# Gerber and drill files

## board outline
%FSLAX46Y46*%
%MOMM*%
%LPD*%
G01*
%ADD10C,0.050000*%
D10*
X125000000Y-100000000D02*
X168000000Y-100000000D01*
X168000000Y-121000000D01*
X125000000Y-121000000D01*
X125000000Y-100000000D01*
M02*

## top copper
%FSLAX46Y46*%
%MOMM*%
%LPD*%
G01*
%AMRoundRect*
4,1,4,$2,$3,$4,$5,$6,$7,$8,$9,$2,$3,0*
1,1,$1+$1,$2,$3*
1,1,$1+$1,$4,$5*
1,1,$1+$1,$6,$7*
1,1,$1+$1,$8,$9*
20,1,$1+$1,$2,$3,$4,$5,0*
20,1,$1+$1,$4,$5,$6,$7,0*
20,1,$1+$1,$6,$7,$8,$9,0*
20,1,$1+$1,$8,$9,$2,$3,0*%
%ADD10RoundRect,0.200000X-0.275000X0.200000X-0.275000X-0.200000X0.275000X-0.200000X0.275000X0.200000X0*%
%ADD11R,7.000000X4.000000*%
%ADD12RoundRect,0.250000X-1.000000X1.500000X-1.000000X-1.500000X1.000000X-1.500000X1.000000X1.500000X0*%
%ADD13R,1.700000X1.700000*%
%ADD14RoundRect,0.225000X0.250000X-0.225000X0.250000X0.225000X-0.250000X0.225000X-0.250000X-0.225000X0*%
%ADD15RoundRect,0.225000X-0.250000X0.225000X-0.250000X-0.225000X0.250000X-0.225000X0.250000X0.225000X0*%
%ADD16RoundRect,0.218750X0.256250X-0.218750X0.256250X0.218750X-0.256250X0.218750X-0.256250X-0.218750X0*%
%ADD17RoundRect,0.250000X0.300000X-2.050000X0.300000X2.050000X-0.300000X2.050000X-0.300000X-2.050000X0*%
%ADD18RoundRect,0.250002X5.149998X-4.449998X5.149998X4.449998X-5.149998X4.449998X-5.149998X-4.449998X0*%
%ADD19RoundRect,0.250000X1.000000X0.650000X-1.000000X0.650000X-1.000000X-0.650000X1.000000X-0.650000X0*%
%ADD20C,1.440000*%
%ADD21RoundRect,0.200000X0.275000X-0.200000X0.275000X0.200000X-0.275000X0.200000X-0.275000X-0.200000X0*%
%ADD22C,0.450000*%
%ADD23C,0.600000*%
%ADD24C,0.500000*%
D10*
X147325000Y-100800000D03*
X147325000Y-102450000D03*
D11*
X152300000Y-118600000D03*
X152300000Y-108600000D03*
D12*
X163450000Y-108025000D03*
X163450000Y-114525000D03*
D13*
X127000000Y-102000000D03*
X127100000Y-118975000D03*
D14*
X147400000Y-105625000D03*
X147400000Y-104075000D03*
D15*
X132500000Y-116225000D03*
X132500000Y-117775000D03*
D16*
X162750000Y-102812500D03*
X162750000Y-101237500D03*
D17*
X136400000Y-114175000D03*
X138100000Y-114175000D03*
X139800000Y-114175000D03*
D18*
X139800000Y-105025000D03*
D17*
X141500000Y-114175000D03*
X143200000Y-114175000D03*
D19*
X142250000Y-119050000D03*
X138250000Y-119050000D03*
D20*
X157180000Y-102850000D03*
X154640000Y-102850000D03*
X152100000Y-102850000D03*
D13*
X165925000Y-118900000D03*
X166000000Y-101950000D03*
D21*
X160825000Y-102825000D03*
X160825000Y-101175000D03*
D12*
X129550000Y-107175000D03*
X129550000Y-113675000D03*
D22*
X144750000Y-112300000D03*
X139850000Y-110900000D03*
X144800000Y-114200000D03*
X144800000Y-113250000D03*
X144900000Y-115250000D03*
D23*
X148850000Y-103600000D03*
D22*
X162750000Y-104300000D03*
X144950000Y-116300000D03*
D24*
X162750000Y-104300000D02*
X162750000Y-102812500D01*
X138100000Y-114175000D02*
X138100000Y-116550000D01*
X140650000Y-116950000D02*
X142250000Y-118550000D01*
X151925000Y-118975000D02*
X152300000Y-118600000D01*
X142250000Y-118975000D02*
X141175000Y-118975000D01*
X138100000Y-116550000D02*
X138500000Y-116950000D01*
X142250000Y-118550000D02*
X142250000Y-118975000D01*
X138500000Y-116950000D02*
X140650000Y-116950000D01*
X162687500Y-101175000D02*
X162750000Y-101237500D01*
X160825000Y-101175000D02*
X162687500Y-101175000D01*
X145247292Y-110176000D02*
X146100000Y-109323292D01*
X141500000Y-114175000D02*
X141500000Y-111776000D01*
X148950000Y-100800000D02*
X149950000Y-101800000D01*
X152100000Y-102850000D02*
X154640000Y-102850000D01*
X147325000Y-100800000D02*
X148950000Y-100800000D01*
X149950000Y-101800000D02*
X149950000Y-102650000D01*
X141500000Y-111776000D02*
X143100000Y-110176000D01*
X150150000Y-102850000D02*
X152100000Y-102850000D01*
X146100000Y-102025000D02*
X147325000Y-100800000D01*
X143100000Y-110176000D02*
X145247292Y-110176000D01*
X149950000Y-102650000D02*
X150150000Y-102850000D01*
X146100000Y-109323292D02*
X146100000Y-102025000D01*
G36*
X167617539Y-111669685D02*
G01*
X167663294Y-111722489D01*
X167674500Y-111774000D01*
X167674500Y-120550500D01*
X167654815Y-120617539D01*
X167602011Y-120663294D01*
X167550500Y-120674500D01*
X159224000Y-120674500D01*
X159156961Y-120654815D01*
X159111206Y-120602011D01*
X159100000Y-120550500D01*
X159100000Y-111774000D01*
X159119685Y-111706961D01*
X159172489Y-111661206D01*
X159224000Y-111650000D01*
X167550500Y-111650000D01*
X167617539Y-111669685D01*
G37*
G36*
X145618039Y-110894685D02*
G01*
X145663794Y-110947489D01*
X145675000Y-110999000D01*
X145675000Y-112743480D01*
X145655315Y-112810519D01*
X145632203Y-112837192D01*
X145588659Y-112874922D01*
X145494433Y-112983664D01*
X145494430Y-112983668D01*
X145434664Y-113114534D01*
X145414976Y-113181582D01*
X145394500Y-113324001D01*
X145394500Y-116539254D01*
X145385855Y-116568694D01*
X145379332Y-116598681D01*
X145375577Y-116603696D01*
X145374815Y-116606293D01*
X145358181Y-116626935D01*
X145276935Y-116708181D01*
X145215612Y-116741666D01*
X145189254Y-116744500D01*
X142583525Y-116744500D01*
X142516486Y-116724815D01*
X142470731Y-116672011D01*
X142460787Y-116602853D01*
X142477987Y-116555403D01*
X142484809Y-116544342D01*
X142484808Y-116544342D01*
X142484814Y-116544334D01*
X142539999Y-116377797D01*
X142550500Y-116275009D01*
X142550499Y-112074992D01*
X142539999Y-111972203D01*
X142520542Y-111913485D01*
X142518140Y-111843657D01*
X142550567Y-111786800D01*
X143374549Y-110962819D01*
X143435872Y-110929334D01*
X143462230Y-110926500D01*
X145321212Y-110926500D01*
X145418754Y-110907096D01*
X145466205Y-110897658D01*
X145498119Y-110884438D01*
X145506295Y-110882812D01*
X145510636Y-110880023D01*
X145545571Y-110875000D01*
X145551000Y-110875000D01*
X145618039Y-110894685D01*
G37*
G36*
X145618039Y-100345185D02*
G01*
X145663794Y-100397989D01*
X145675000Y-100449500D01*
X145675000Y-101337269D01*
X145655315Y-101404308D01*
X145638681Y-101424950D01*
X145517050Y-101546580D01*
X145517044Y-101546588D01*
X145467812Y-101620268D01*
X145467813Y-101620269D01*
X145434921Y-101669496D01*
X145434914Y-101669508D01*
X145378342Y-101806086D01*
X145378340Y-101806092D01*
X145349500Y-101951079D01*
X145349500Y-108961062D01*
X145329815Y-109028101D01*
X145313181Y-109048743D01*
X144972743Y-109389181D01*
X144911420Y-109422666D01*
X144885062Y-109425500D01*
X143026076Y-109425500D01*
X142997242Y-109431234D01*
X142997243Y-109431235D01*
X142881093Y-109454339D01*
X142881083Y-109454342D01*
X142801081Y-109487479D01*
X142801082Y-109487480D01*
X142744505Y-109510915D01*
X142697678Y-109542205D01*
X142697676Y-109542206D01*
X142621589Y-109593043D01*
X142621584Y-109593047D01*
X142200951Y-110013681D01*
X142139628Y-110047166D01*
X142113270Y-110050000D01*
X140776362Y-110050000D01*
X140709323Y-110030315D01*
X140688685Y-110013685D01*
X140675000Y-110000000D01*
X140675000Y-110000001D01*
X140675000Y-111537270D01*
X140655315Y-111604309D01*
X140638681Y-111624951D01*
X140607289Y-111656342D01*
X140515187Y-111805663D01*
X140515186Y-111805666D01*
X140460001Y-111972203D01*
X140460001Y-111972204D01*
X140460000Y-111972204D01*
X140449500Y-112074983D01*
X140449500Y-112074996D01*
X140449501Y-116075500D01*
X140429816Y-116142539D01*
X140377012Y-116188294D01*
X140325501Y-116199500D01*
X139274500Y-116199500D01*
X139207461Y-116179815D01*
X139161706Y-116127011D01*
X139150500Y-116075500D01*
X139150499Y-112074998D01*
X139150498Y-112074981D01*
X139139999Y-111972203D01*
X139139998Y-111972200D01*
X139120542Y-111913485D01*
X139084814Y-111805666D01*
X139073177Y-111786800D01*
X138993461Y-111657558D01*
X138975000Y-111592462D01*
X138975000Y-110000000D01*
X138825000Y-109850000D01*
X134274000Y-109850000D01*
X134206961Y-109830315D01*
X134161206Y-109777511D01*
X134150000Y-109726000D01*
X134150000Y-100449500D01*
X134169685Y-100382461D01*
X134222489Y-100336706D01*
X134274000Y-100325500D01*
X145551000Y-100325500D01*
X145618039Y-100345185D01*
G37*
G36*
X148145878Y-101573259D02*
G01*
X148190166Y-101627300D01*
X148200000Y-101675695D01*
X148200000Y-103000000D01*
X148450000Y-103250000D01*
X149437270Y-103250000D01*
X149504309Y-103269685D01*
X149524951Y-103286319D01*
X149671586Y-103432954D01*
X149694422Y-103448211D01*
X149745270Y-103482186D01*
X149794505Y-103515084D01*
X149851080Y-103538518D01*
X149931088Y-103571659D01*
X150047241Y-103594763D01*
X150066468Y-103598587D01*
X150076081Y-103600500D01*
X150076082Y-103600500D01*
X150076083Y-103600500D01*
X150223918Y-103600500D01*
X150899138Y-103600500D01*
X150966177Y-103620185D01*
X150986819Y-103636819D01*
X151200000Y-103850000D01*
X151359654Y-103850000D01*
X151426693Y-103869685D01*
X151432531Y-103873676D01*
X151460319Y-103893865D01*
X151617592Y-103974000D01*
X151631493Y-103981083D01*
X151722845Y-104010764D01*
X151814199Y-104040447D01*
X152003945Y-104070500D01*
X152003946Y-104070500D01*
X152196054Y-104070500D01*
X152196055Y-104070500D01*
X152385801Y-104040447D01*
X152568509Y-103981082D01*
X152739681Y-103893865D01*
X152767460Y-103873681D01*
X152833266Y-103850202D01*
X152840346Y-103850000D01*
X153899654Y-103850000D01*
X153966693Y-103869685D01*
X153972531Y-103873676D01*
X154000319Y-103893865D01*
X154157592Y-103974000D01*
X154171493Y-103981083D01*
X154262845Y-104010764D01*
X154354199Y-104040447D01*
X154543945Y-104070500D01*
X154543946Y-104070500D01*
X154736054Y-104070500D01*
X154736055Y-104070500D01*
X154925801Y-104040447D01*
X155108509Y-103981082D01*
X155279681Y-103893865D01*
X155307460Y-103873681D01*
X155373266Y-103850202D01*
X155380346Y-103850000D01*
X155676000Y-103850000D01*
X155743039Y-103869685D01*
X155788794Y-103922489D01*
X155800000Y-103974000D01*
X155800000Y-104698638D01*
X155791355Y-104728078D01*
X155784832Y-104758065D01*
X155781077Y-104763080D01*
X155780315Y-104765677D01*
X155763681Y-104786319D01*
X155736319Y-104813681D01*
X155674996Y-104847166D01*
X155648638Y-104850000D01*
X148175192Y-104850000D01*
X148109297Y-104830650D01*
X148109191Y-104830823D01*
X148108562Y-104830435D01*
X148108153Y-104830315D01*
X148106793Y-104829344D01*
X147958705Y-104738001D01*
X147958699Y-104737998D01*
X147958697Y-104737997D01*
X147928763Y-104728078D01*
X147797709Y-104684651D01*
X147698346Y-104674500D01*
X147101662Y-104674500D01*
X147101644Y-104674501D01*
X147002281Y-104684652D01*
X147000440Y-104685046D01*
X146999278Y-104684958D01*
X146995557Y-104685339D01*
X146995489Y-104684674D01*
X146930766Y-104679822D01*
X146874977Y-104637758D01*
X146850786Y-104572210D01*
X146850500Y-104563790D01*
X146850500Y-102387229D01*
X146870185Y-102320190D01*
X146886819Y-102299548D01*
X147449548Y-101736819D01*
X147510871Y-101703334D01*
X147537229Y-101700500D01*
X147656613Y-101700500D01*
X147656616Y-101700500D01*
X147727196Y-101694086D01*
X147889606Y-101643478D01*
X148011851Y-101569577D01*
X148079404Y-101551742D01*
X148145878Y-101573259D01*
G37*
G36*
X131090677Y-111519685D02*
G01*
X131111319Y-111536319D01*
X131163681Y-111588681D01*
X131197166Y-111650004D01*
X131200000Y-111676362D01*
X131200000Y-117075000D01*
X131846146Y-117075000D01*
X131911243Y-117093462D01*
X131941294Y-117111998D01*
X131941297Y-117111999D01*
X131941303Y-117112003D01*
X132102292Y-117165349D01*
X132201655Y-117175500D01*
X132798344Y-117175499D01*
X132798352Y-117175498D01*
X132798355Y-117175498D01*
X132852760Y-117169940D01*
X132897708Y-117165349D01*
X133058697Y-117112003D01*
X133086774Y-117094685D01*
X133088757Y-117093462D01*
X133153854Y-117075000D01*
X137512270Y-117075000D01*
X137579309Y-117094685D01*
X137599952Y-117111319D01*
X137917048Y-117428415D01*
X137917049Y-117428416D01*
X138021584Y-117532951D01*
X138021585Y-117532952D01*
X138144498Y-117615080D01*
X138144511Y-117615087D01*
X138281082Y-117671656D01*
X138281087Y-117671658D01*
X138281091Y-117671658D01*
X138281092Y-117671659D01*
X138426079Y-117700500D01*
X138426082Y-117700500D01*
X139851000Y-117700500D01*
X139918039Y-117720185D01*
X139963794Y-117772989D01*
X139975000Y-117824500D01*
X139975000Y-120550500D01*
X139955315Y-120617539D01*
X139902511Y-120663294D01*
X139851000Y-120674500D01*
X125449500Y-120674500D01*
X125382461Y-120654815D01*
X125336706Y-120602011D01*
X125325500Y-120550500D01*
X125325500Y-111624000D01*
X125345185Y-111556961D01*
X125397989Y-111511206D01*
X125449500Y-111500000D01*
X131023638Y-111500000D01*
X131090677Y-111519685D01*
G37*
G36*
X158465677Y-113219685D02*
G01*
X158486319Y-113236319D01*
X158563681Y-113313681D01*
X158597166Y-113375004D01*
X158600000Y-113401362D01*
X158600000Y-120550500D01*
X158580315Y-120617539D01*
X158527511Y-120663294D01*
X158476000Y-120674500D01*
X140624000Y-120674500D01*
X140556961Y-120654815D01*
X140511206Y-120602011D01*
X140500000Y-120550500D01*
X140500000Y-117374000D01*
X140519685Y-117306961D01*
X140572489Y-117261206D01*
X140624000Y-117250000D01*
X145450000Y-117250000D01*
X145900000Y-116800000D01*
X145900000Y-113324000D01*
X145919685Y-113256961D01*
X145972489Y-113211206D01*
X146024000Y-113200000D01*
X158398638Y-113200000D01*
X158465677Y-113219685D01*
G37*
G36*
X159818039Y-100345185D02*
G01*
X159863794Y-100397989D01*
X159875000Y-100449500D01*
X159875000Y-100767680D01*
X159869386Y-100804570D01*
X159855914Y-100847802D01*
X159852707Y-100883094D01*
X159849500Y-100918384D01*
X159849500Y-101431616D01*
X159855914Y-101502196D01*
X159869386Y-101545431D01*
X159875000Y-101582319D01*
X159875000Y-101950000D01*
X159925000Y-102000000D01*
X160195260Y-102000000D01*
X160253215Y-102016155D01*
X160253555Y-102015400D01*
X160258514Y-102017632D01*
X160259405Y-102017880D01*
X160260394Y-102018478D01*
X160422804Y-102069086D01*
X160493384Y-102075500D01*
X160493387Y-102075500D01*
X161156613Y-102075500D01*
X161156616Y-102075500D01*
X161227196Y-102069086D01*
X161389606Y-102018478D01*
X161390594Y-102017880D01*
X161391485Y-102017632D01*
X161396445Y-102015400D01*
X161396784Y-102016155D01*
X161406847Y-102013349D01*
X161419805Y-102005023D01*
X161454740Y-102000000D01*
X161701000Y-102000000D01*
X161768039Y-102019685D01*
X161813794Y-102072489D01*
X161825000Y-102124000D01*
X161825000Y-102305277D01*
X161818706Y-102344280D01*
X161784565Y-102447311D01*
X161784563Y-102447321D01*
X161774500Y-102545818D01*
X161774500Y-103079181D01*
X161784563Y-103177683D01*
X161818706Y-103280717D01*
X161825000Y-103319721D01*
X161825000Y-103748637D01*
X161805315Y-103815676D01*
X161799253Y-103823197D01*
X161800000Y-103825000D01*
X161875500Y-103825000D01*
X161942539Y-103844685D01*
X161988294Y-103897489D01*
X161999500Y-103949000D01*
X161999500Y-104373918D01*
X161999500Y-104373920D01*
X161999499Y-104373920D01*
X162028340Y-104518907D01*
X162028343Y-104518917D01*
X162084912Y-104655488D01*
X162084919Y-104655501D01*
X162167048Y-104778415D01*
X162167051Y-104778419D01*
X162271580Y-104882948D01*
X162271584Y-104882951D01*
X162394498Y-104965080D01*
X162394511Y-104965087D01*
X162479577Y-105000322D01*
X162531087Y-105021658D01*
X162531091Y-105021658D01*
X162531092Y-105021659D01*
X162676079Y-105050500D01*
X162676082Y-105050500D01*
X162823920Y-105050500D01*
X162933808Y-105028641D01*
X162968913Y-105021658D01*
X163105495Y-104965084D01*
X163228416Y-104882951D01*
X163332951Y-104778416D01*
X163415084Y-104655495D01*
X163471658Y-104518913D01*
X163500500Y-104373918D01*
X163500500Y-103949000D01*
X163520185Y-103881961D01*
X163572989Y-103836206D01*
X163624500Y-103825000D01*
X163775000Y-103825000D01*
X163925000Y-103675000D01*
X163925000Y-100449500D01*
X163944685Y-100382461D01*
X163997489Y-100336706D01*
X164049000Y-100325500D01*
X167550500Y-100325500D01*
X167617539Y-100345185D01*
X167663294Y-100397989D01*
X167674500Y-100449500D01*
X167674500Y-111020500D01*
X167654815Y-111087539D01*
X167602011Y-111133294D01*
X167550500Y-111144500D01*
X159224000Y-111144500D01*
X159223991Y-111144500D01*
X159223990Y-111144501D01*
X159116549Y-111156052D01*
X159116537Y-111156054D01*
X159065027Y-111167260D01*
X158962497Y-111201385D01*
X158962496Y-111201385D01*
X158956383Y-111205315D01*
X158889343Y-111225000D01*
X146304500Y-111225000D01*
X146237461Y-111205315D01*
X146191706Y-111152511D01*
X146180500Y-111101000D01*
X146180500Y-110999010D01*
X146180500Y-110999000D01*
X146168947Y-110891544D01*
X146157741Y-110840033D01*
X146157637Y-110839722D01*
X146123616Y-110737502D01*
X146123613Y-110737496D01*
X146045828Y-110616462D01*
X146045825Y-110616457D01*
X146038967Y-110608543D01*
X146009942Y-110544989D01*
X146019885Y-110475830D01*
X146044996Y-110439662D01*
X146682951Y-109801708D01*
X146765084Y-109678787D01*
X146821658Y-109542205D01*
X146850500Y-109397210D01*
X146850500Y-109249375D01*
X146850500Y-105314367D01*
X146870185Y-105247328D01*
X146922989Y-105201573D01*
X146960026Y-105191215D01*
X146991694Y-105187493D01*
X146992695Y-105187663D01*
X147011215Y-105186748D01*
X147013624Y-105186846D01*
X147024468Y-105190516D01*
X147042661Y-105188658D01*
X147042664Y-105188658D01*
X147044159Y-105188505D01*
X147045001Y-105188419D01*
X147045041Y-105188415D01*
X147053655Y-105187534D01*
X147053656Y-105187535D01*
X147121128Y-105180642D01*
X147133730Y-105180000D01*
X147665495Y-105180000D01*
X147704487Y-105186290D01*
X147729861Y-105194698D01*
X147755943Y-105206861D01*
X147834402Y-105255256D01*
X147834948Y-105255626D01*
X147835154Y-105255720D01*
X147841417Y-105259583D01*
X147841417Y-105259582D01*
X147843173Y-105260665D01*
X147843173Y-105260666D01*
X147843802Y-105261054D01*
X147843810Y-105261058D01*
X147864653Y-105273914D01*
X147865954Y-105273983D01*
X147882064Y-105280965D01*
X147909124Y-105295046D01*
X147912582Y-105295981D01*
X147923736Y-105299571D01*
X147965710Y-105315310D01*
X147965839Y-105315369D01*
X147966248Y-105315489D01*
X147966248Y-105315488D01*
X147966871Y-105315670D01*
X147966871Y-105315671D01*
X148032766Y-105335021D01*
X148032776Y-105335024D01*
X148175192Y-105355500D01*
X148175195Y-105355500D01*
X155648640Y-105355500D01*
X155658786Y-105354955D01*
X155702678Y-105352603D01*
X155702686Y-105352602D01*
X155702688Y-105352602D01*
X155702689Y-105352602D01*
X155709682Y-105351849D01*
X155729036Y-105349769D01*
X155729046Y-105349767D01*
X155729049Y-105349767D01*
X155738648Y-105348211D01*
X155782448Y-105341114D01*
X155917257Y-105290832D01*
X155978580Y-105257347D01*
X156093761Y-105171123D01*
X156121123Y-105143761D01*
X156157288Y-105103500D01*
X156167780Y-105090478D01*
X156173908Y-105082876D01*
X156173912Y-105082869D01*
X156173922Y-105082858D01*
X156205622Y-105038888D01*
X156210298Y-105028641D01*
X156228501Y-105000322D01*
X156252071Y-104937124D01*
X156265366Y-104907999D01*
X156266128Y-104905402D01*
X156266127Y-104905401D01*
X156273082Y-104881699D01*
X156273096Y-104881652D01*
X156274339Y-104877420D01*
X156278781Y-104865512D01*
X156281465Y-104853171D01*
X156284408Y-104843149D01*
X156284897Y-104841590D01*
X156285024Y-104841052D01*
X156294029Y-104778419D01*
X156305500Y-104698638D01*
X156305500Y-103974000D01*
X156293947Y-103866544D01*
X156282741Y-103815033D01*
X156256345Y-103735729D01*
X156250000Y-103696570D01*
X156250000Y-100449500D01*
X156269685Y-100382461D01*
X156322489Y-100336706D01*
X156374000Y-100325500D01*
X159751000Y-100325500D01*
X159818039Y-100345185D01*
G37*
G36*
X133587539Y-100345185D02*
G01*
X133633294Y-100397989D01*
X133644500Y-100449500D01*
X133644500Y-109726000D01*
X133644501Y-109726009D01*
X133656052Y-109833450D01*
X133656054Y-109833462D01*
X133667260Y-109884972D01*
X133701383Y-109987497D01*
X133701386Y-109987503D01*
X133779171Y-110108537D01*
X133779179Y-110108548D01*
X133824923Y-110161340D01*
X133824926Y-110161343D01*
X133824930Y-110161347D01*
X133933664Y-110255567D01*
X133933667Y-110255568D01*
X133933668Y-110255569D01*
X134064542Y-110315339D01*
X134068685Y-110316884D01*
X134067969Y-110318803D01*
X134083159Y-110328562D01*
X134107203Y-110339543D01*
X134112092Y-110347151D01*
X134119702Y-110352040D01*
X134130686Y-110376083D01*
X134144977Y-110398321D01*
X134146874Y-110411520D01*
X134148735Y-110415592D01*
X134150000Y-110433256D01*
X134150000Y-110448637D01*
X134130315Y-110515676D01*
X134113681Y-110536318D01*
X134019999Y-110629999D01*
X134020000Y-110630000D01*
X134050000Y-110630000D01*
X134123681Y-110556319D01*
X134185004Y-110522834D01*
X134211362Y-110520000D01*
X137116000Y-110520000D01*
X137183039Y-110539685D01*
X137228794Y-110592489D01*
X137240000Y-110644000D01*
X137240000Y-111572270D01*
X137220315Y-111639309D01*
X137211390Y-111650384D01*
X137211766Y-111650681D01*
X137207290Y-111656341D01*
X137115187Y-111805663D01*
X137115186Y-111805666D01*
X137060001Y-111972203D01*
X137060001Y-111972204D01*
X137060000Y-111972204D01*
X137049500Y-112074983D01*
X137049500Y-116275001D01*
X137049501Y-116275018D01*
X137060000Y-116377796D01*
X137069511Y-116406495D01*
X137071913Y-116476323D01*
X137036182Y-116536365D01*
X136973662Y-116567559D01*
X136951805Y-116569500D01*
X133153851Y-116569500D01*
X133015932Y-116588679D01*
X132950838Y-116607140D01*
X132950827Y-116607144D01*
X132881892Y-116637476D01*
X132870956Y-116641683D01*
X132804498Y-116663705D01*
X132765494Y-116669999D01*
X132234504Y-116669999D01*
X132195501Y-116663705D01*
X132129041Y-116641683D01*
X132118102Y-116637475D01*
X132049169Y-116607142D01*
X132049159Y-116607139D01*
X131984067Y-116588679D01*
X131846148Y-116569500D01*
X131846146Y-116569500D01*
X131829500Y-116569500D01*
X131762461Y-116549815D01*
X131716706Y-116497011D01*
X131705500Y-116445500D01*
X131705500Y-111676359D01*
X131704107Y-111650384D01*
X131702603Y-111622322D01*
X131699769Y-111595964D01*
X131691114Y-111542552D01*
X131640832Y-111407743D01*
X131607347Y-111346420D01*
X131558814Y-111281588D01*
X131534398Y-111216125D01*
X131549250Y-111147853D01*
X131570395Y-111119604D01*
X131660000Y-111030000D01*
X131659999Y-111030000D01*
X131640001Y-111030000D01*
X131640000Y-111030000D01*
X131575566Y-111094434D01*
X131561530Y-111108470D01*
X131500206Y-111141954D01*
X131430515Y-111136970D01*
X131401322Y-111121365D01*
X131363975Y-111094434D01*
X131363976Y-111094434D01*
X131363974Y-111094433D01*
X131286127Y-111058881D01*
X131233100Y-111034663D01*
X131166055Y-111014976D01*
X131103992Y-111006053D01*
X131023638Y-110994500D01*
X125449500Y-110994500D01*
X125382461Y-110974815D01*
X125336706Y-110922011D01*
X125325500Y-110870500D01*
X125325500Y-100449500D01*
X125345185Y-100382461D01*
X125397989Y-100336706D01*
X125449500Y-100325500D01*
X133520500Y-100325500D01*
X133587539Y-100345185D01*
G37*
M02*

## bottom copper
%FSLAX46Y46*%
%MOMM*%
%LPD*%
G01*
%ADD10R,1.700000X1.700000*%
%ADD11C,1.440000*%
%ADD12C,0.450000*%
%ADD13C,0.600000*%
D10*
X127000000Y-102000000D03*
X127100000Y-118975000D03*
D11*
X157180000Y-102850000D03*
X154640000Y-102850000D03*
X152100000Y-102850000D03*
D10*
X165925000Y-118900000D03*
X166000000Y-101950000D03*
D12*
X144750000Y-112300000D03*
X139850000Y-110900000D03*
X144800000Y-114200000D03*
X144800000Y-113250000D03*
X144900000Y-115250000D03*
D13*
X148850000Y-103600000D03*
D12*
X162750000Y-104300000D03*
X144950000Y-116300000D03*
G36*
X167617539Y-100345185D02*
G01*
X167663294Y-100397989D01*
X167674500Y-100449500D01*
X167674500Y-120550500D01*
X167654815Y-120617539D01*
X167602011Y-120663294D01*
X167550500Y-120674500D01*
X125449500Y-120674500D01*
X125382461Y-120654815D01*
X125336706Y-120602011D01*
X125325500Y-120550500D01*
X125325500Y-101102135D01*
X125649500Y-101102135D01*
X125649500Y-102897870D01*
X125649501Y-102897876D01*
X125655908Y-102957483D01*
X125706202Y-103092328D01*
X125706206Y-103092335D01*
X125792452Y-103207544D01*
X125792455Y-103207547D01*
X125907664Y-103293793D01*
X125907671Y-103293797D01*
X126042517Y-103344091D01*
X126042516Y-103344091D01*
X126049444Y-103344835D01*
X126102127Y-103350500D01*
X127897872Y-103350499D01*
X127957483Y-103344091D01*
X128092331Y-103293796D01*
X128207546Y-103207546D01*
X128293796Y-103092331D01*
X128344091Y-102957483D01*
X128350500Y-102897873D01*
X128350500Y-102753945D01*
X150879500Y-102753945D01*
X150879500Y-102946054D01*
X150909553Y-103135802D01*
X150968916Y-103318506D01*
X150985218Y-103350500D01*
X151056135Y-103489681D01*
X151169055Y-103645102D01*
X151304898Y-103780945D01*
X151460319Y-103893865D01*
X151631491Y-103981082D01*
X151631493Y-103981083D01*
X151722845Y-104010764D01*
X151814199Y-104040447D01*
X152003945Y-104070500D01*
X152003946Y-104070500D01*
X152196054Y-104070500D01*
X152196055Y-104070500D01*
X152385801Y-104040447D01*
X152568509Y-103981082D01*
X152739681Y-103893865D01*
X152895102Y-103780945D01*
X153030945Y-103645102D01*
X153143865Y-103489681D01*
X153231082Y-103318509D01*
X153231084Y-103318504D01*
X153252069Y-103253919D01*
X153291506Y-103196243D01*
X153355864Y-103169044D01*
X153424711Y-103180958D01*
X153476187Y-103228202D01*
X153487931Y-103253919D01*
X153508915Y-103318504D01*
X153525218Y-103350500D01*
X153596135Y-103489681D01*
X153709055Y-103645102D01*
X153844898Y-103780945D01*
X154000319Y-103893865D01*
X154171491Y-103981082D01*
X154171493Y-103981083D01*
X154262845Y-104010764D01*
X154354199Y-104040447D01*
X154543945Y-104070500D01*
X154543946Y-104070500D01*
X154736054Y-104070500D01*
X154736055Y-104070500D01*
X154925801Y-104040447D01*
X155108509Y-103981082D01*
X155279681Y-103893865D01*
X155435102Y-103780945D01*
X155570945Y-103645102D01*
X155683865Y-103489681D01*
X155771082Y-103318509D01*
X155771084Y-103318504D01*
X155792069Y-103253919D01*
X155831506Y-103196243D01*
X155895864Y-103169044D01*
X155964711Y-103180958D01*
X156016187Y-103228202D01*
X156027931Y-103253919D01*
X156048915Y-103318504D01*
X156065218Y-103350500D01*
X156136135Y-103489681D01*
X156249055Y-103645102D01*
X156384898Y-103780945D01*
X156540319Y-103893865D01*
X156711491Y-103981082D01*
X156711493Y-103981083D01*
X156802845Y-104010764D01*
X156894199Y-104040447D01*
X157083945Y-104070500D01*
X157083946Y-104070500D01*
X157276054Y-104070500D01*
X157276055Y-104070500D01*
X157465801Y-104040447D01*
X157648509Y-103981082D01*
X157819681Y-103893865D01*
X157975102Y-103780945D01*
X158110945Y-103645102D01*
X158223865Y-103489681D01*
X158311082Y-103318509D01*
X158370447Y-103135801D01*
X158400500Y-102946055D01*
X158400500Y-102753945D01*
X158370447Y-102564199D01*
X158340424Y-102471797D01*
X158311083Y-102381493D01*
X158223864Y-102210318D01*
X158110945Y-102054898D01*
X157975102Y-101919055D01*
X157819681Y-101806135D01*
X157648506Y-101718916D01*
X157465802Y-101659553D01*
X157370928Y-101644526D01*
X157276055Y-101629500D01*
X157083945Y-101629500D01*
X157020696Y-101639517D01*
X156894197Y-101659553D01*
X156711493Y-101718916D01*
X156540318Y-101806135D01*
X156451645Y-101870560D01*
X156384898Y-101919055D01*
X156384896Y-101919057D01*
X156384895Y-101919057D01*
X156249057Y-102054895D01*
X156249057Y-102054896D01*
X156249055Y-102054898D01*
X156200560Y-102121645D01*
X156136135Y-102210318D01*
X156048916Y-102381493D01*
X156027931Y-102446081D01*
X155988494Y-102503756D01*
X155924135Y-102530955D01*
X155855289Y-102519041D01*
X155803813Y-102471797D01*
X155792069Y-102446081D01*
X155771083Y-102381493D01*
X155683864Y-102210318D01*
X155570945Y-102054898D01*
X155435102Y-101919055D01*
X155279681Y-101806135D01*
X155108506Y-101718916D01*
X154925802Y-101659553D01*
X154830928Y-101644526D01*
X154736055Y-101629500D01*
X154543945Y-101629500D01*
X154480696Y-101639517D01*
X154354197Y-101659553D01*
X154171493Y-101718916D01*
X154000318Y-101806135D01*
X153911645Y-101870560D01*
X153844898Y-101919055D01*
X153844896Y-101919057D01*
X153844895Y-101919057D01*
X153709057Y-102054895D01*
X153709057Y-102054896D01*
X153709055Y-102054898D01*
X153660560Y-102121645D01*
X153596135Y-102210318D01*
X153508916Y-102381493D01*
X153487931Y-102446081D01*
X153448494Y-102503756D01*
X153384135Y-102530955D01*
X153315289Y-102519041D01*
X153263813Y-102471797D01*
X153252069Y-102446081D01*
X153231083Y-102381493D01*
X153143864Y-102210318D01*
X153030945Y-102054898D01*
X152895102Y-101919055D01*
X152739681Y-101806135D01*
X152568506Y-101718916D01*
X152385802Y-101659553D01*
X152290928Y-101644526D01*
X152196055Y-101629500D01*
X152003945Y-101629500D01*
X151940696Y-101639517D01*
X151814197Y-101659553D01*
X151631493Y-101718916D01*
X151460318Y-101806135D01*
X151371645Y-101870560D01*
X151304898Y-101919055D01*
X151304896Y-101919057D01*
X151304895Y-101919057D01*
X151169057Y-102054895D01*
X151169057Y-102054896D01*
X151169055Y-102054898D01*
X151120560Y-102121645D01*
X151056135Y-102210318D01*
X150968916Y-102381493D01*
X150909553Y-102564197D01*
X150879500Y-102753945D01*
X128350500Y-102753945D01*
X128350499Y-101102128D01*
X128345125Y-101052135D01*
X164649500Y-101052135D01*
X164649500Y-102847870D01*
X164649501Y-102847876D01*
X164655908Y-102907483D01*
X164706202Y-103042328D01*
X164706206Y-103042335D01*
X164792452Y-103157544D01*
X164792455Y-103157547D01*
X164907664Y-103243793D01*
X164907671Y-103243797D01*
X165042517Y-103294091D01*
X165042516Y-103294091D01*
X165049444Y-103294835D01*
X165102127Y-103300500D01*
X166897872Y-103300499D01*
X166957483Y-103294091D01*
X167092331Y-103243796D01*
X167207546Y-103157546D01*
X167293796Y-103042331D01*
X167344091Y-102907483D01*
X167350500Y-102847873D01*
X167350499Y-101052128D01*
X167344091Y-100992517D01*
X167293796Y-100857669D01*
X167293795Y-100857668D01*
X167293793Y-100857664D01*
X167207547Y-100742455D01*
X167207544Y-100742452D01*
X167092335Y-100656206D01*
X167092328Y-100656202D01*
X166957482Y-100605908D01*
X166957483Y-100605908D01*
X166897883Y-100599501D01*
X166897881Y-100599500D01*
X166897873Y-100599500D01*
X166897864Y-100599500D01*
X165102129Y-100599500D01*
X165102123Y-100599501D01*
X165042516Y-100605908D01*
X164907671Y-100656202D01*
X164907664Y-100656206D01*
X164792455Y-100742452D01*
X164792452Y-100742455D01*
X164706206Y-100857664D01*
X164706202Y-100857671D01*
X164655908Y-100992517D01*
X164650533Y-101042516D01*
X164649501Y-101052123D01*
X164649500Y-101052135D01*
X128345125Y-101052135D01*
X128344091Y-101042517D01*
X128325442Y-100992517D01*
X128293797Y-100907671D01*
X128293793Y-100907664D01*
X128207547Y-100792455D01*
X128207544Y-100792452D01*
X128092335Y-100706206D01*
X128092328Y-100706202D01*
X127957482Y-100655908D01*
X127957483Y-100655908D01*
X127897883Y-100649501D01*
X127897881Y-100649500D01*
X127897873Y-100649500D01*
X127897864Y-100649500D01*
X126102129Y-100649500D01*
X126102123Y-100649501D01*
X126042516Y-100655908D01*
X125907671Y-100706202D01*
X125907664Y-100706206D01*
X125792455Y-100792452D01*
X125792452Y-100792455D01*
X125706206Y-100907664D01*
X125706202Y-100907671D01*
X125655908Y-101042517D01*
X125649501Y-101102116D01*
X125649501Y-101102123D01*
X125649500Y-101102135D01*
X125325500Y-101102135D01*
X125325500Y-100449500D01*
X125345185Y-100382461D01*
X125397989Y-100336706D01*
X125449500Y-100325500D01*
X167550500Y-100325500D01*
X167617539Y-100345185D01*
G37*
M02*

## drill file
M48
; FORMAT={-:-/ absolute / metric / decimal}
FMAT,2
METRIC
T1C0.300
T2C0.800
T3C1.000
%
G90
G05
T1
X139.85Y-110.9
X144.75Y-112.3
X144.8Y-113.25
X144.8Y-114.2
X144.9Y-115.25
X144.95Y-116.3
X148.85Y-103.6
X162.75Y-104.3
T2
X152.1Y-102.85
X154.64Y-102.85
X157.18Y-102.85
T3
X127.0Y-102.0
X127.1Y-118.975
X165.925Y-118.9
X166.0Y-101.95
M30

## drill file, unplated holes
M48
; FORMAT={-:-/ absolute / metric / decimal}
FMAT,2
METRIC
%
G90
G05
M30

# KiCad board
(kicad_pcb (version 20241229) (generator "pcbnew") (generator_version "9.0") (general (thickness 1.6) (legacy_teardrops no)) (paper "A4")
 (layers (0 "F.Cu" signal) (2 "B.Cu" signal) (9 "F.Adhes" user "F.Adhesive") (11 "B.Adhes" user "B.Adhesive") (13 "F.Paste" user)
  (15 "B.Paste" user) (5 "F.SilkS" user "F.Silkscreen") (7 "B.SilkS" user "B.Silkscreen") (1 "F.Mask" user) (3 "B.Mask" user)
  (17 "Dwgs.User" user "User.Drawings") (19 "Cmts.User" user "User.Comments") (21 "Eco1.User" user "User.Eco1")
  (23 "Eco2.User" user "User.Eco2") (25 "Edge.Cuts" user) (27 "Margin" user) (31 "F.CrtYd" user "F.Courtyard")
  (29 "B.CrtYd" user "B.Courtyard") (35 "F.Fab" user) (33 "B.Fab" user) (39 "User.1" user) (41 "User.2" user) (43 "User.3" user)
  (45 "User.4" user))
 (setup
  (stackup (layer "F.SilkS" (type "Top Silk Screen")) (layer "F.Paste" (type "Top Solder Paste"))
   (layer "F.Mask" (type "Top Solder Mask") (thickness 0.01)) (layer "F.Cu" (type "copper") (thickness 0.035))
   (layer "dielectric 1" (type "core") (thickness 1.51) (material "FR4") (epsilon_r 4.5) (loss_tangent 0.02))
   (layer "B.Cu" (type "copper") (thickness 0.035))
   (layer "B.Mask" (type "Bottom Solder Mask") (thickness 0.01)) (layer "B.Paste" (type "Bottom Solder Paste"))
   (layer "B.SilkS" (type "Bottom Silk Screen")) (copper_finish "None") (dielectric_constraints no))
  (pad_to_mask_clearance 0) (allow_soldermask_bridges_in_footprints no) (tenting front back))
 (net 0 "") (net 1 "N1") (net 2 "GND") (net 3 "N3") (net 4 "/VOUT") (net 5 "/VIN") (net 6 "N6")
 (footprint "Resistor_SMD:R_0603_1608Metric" (layer "F.Cu") (at 147.325 101.625 -90)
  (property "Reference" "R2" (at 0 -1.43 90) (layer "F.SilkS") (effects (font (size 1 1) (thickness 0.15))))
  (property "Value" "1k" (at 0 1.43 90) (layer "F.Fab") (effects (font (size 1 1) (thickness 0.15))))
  (pad "1" smd roundrect (at -0.825 0 270) (size 0.8 0.95) (layers "F.Cu" "F.Mask" "F.Paste") (roundrect_rratio 0.25) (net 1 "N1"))
  (pad "2" smd roundrect (at 0.825 0 270) (size 0.8 0.95) (layers "F.Cu" "F.Mask" "F.Paste") (roundrect_rratio 0.25) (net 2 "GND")))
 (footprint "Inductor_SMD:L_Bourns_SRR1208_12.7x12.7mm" (layer "F.Cu") (at 152.3 113.6 90)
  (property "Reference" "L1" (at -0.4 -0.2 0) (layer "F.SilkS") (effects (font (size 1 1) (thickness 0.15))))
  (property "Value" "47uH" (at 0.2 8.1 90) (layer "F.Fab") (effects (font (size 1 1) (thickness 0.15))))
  (pad "1" smd rect (at -5 0 90) (size 4 7) (layers "F.Cu" "F.Mask" "F.Paste") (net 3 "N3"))
  (pad "2" smd rect (at 5 0 90) (size 4 7) (layers "F.Cu" "F.Mask" "F.Paste") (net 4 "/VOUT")))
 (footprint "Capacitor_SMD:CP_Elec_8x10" (layer "F.Cu") (at 163.45 111.275 -90)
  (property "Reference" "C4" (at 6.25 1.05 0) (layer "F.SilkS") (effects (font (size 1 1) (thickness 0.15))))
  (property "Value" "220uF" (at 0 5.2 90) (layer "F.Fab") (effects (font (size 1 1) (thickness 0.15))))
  (pad "1" smd roundrect (at -3.25 0 270) (size 3.5 2.5) (layers "F.Cu" "F.Mask" "F.Paste") (roundrect_rratio 0.1) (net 4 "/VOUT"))
  (pad "2" smd roundrect (at 3.25 0 270) (size 3.5 2.5) (layers "F.Cu" "F.Mask" "F.Paste") (roundrect_rratio 0.1) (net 2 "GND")))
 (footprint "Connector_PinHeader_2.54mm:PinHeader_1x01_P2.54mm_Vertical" (layer "F.Cu") (at 127 102)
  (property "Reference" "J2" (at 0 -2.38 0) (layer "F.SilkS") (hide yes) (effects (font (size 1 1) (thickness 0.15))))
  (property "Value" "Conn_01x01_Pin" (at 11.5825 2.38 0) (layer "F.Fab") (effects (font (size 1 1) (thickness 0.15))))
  (pad "1" thru_hole rect (at 0 0) (size 1.7 1.7) (drill 1) (layers "*.Cu" "*.Mask") (remove_unused_layers no) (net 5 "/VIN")))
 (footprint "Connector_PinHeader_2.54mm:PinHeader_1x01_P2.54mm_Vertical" (layer "F.Cu") (at 127.1 118.975)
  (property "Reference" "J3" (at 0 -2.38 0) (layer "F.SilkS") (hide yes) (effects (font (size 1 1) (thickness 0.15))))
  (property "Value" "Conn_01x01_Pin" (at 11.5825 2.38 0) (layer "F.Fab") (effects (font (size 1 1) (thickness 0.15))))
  (pad "1" thru_hole rect (at 0 0) (size 1.7 1.7) (drill 1) (layers "*.Cu" "*.Mask") (remove_unused_layers no) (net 2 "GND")))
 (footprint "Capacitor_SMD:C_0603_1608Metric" (layer "F.Cu") (at 147.4 104.85 90)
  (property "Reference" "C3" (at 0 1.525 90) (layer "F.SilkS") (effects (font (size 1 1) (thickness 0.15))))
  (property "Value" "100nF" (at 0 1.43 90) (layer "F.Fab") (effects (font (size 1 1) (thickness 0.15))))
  (pad "1" smd roundrect (at -0.775 0 90) (size 0.9 0.95) (layers "F.Cu" "F.Mask" "F.Paste") (roundrect_rratio 0.25) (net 4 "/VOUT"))
  (pad "2" smd roundrect (at 0.775 0 90) (size 0.9 0.95) (layers "F.Cu" "F.Mask" "F.Paste") (roundrect_rratio 0.25) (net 2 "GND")))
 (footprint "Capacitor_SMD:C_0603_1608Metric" (layer "F.Cu") (at 132.5 117 -90)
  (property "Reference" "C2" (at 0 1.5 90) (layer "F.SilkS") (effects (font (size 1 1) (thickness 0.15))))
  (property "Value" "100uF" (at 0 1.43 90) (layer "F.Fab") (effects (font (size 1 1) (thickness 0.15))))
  (pad "1" smd roundrect (at -0.775 0 270) (size 0.9 0.95) (layers "F.Cu" "F.Mask" "F.Paste") (roundrect_rratio 0.25) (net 5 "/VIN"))
  (pad "2" smd roundrect (at 0.775 0 270) (size 0.9 0.95) (layers "F.Cu" "F.Mask" "F.Paste") (roundrect_rratio 0.25) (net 2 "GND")))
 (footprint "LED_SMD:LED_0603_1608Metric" (layer "F.Cu") (at 162.75 102.025 90)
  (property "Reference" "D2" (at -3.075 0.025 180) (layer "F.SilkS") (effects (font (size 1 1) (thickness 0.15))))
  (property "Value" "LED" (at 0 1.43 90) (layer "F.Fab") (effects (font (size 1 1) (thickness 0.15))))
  (pad "1" smd roundrect (at -0.7875 0 90) (size 0.875 0.95) (layers "F.Cu" "F.Mask" "F.Paste") (roundrect_rratio 0.25) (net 2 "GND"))
  (pad "2" smd roundrect (at 0.7875 0 90) (size 0.875 0.95) (layers "F.Cu" "F.Mask" "F.Paste") (roundrect_rratio 0.25) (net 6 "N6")))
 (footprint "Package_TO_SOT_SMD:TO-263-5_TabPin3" (layer "F.Cu") (at 139.8 106.525 90)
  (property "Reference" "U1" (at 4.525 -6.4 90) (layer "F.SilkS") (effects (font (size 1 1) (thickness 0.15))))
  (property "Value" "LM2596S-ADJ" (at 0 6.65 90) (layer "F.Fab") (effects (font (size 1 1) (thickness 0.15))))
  (pad "" smd roundrect (at -0.925 -2.775 90) (size 4.55 5.25) (layers "F.Paste") (roundrect_rratio 0.054945))
  (pad "" smd roundrect (at -0.925 2.775 90) (size 4.55 5.25) (layers "F.Paste") (roundrect_rratio 0.054945))
  (pad "" smd roundrect (at 3.925 -2.775 90) (size 4.55 5.25) (layers "F.Paste") (roundrect_rratio 0.054945))
  (pad "" smd roundrect (at 3.925 2.775 90) (size 4.55 5.25) (layers "F.Paste") (roundrect_rratio 0.054945))
  (pad "1" smd roundrect (at -7.65 -3.4 90) (size 4.6 1.1) (layers "F.Cu" "F.Mask" "F.Paste") (roundrect_rratio 0.227273) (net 5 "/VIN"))
  (pad "2" smd roundrect (at -7.65 -1.7 90) (size 4.6 1.1) (layers "F.Cu" "F.Mask" "F.Paste") (roundrect_rratio 0.227273) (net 3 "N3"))
  (pad "3" smd roundrect (at -7.65 0 90) (size 4.6 1.1) (layers "F.Cu" "F.Mask" "F.Paste") (roundrect_rratio 0.227273) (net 2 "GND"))
  (pad "3" smd roundrect (at 1.5 0 90) (size 9.4 10.8) (layers "F.Cu" "F.Mask") (roundrect_rratio 0.026596) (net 2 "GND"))
  (pad "4" smd roundrect (at -7.65 1.7 90) (size 4.6 1.1) (layers "F.Cu" "F.Mask" "F.Paste") (roundrect_rratio 0.227273) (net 1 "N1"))
  (pad "5" smd roundrect (at -7.65 3.4 90) (size 4.6 1.1) (layers "F.Cu" "F.Mask" "F.Paste") (roundrect_rratio 0.227273) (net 2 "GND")))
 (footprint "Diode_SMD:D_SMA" (layer "F.Cu") (at 140.25 119.05 180)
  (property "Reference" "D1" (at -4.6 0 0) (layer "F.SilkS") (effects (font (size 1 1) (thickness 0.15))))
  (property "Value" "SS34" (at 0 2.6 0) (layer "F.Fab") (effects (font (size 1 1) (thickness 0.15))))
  (pad "1" smd roundrect (at -2 0 180) (size 2.5 1.8) (layers "F.Cu" "F.Mask" "F.Paste") (roundrect_rratio 0.1388888889) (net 3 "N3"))
  (pad "2" smd roundrect (at 2 0 180) (size 2.5 1.8) (layers "F.Cu" "F.Mask" "F.Paste") (roundrect_rratio 0.1388888889) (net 2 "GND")))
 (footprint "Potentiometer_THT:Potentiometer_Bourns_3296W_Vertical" (layer "F.Cu") (at 157.18 102.85)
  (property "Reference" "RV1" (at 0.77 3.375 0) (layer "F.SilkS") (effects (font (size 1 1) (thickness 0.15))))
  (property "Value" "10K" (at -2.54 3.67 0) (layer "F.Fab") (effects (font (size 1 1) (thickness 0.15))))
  (pad "1" thru_hole circle (at 0 0) (size 1.44 1.44) (drill 0.8) (layers "*.Cu" "*.Mask") (remove_unused_layers no) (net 4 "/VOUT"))
  (pad "2" thru_hole circle (at -2.54 0) (size 1.44 1.44) (drill 0.8) (layers "*.Cu" "*.Mask") (remove_unused_layers no) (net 1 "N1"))
  (pad "3" thru_hole circle (at -5.08 0) (size 1.44 1.44) (drill 0.8) (layers "*.Cu" "*.Mask") (remove_unused_layers no) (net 1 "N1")))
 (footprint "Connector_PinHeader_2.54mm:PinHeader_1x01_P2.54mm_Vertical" (layer "F.Cu") (at 165.925 118.9)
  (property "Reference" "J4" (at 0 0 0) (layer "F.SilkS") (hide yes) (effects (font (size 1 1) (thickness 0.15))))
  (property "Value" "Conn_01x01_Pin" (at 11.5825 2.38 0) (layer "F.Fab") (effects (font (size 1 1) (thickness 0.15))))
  (pad "1" thru_hole rect (at 0 0) (size 1.7 1.7) (drill 1) (layers "*.Cu" "*.Mask") (remove_unused_layers no) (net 2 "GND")))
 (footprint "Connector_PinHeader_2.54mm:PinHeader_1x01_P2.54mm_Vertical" (layer "F.Cu") (at 166 101.95)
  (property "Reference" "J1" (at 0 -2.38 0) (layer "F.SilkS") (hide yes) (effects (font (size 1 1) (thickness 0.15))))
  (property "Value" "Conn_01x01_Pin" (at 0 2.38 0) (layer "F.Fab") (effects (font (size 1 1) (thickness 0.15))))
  (pad "1" thru_hole rect (at 0 0) (size 1.7 1.7) (drill 1) (layers "*.Cu" "*.Mask") (remove_unused_layers no) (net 4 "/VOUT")))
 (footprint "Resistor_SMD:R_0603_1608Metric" (layer "F.Cu") (at 160.825 102 90)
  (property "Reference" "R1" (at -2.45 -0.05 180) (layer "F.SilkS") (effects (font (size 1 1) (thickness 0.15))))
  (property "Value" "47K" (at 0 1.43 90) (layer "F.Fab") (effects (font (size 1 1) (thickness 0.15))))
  (pad "1" smd roundrect (at -0.825 0 90) (size 0.8 0.95) (layers "F.Cu" "F.Mask" "F.Paste") (roundrect_rratio 0.25) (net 4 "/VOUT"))
  (pad "2" smd roundrect (at 0.825 0 90) (size 0.8 0.95) (layers "F.Cu" "F.Mask" "F.Paste") (roundrect_rratio 0.25) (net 6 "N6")))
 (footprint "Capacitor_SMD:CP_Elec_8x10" (layer "F.Cu") (at 129.55 110.425 -90)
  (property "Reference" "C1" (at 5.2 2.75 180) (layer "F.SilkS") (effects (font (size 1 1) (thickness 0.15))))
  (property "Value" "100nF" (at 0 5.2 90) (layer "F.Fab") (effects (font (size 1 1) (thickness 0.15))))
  (pad "1" smd roundrect (at -3.25 0 270) (size 3.5 2.5) (layers "F.Cu" "F.Mask" "F.Paste") (roundrect_rratio 0.1) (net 5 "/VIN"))
  (pad "2" smd roundrect (at 3.25 0 270) (size 3.5 2.5) (layers "F.Cu" "F.Mask" "F.Paste") (roundrect_rratio 0.1) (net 2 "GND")))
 (gr_rect (start 125 100) (end 168 121) (stroke (width 0.05) (type default)) (fill no) (layer "Edge.Cuts"))
 (segment (start 162.75 104.3) (end 162.75 102.8125) (width 0.5) (layer "F.Cu") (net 2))
 (via (at 144.75 112.3) (size 0.45) (drill 0.3) (layers "F.Cu" "B.Cu") (free yes) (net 2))
 (via (at 139.85 110.9) (size 0.45) (drill 0.3) (layers "F.Cu" "B.Cu") (free yes) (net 2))
 (via (at 144.8 114.2) (size 0.45) (drill 0.3) (layers "F.Cu" "B.Cu") (free yes) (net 2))
 (via (at 144.8 113.25) (size 0.45) (drill 0.3) (layers "F.Cu" "B.Cu") (free yes) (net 2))
 (via (at 144.9 115.25) (size 0.45) (drill 0.3) (layers "F.Cu" "B.Cu") (free yes) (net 2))
 (via (at 148.85 103.6) (size 0.6) (drill 0.3) (layers "F.Cu" "B.Cu") (free yes) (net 2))
 (via (at 162.75 104.3) (size 0.45) (drill 0.3) (layers "F.Cu" "B.Cu") (free yes) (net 2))
 (via (at 144.95 116.3) (size 0.45) (drill 0.3) (layers "F.Cu" "B.Cu") (free yes) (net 2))
 (segment (start 138.1 114.175) (end 138.1 116.55) (width 0.5) (layer "F.Cu") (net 3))
 (segment (start 140.65 116.95) (end 142.25 118.55) (width 0.5) (layer "F.Cu") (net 3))
 (segment (start 151.925 118.975) (end 152.3 118.6) (width 0.5) (layer "F.Cu") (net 3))
 (segment (start 142.25 118.975) (end 141.175 118.975) (width 0.5) (layer "F.Cu") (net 3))
 (segment (start 138.1 116.55) (end 138.5 116.95) (width 0.5) (layer "F.Cu") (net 3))
 (segment (start 142.25 118.55) (end 142.25 118.975) (width 0.5) (layer "F.Cu") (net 3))
 (segment (start 138.5 116.95) (end 140.65 116.95) (width 0.5) (layer "F.Cu") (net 3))
 (segment (start 162.6875 101.175) (end 162.75 101.2375) (width 0.5) (layer "F.Cu") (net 6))
 (segment (start 160.825 101.175) (end 162.6875 101.175) (width 0.5) (layer "F.Cu") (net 6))
 (segment (start 145.247292 110.176) (end 146.1 109.323292) (width 0.5) (layer "F.Cu") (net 1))
 (segment (start 141.5 114.175) (end 141.5 111.776) (width 0.5) (layer "F.Cu") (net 1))
 (segment (start 148.95 100.8) (end 149.95 101.8) (width 0.5) (layer "F.Cu") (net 1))
 (segment (start 152.1 102.85) (end 154.64 102.85) (width 0.5) (layer "F.Cu") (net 1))
 (segment (start 147.325 100.8) (end 148.95 100.8) (width 0.5) (layer "F.Cu") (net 1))
 (segment (start 149.95 101.8) (end 149.95 102.65) (width 0.5) (layer "F.Cu") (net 1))
 (segment (start 141.5 111.776) (end 143.1 110.176) (width 0.5) (layer "F.Cu") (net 1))
 (segment (start 150.15 102.85) (end 152.1 102.85) (width 0.5) (layer "F.Cu") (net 1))
 (segment (start 146.1 102.025) (end 147.325 100.8) (width 0.5) (layer "F.Cu") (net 1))
 (segment (start 143.1 110.176) (end 145.247292 110.176) (width 0.5) (layer "F.Cu") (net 1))
 (segment (start 149.95 102.65) (end 150.15 102.85) (width 0.5) (layer "F.Cu") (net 1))
 (segment (start 146.1 109.323292) (end 146.1 102.025) (width 0.5) (layer "F.Cu") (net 1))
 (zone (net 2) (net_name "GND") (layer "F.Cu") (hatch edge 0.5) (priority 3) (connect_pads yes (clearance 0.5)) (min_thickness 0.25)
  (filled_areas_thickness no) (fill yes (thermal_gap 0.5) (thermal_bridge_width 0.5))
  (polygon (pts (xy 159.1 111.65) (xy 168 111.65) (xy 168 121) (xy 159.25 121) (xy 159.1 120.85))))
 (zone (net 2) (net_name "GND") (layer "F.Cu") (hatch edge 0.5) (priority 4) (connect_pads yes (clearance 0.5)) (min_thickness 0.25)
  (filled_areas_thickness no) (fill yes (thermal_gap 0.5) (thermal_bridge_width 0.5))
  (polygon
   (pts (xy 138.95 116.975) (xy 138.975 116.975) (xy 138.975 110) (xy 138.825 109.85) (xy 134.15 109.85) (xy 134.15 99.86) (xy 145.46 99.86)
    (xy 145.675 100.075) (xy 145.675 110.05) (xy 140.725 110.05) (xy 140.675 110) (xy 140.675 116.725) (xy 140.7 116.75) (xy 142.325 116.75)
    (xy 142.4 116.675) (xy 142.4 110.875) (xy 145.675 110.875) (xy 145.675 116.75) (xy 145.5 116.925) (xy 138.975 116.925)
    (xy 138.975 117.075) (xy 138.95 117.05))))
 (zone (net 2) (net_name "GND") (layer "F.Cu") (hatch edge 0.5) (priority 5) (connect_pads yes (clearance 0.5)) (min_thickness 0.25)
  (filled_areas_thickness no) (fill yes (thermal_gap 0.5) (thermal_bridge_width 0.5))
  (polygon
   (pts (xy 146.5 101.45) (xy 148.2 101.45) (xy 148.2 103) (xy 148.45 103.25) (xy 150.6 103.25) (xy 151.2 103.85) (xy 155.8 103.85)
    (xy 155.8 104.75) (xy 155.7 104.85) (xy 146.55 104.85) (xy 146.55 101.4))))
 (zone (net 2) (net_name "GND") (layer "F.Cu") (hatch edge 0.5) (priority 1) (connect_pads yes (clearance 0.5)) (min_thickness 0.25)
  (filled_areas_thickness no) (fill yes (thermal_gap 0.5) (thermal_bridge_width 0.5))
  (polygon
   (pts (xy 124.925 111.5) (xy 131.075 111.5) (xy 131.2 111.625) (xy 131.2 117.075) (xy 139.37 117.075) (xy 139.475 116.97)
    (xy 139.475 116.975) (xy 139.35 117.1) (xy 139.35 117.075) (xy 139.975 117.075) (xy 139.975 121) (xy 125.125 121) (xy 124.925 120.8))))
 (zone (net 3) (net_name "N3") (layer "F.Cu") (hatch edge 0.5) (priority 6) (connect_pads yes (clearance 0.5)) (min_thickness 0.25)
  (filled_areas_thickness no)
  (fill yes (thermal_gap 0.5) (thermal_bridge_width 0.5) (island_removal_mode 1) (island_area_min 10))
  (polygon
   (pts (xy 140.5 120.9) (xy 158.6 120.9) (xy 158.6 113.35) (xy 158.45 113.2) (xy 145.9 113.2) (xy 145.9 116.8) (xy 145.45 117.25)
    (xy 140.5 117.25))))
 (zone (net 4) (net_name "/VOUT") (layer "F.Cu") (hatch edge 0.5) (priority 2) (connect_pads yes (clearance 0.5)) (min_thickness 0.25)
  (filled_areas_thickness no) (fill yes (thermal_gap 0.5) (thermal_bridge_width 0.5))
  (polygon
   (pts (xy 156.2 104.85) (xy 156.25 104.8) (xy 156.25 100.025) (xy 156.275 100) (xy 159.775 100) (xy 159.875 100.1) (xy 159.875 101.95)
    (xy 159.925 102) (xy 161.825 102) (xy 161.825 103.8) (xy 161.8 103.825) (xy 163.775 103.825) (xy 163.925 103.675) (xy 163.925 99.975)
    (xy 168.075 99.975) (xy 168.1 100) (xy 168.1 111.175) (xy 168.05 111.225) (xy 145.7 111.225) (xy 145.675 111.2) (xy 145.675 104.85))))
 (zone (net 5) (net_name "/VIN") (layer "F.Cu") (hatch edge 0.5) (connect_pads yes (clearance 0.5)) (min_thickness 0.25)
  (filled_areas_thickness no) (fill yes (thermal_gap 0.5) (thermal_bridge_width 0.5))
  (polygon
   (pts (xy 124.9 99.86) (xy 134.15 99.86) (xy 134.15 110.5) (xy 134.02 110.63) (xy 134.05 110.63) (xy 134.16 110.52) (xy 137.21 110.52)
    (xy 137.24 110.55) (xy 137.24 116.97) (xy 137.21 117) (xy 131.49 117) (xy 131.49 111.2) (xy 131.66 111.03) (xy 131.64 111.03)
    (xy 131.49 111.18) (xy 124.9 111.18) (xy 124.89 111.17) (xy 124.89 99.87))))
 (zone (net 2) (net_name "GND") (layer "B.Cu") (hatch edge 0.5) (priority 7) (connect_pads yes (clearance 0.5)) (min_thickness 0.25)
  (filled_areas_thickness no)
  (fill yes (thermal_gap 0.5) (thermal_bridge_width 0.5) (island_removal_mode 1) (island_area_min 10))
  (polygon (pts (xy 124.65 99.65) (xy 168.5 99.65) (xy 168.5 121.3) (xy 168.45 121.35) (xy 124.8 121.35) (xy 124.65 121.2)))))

